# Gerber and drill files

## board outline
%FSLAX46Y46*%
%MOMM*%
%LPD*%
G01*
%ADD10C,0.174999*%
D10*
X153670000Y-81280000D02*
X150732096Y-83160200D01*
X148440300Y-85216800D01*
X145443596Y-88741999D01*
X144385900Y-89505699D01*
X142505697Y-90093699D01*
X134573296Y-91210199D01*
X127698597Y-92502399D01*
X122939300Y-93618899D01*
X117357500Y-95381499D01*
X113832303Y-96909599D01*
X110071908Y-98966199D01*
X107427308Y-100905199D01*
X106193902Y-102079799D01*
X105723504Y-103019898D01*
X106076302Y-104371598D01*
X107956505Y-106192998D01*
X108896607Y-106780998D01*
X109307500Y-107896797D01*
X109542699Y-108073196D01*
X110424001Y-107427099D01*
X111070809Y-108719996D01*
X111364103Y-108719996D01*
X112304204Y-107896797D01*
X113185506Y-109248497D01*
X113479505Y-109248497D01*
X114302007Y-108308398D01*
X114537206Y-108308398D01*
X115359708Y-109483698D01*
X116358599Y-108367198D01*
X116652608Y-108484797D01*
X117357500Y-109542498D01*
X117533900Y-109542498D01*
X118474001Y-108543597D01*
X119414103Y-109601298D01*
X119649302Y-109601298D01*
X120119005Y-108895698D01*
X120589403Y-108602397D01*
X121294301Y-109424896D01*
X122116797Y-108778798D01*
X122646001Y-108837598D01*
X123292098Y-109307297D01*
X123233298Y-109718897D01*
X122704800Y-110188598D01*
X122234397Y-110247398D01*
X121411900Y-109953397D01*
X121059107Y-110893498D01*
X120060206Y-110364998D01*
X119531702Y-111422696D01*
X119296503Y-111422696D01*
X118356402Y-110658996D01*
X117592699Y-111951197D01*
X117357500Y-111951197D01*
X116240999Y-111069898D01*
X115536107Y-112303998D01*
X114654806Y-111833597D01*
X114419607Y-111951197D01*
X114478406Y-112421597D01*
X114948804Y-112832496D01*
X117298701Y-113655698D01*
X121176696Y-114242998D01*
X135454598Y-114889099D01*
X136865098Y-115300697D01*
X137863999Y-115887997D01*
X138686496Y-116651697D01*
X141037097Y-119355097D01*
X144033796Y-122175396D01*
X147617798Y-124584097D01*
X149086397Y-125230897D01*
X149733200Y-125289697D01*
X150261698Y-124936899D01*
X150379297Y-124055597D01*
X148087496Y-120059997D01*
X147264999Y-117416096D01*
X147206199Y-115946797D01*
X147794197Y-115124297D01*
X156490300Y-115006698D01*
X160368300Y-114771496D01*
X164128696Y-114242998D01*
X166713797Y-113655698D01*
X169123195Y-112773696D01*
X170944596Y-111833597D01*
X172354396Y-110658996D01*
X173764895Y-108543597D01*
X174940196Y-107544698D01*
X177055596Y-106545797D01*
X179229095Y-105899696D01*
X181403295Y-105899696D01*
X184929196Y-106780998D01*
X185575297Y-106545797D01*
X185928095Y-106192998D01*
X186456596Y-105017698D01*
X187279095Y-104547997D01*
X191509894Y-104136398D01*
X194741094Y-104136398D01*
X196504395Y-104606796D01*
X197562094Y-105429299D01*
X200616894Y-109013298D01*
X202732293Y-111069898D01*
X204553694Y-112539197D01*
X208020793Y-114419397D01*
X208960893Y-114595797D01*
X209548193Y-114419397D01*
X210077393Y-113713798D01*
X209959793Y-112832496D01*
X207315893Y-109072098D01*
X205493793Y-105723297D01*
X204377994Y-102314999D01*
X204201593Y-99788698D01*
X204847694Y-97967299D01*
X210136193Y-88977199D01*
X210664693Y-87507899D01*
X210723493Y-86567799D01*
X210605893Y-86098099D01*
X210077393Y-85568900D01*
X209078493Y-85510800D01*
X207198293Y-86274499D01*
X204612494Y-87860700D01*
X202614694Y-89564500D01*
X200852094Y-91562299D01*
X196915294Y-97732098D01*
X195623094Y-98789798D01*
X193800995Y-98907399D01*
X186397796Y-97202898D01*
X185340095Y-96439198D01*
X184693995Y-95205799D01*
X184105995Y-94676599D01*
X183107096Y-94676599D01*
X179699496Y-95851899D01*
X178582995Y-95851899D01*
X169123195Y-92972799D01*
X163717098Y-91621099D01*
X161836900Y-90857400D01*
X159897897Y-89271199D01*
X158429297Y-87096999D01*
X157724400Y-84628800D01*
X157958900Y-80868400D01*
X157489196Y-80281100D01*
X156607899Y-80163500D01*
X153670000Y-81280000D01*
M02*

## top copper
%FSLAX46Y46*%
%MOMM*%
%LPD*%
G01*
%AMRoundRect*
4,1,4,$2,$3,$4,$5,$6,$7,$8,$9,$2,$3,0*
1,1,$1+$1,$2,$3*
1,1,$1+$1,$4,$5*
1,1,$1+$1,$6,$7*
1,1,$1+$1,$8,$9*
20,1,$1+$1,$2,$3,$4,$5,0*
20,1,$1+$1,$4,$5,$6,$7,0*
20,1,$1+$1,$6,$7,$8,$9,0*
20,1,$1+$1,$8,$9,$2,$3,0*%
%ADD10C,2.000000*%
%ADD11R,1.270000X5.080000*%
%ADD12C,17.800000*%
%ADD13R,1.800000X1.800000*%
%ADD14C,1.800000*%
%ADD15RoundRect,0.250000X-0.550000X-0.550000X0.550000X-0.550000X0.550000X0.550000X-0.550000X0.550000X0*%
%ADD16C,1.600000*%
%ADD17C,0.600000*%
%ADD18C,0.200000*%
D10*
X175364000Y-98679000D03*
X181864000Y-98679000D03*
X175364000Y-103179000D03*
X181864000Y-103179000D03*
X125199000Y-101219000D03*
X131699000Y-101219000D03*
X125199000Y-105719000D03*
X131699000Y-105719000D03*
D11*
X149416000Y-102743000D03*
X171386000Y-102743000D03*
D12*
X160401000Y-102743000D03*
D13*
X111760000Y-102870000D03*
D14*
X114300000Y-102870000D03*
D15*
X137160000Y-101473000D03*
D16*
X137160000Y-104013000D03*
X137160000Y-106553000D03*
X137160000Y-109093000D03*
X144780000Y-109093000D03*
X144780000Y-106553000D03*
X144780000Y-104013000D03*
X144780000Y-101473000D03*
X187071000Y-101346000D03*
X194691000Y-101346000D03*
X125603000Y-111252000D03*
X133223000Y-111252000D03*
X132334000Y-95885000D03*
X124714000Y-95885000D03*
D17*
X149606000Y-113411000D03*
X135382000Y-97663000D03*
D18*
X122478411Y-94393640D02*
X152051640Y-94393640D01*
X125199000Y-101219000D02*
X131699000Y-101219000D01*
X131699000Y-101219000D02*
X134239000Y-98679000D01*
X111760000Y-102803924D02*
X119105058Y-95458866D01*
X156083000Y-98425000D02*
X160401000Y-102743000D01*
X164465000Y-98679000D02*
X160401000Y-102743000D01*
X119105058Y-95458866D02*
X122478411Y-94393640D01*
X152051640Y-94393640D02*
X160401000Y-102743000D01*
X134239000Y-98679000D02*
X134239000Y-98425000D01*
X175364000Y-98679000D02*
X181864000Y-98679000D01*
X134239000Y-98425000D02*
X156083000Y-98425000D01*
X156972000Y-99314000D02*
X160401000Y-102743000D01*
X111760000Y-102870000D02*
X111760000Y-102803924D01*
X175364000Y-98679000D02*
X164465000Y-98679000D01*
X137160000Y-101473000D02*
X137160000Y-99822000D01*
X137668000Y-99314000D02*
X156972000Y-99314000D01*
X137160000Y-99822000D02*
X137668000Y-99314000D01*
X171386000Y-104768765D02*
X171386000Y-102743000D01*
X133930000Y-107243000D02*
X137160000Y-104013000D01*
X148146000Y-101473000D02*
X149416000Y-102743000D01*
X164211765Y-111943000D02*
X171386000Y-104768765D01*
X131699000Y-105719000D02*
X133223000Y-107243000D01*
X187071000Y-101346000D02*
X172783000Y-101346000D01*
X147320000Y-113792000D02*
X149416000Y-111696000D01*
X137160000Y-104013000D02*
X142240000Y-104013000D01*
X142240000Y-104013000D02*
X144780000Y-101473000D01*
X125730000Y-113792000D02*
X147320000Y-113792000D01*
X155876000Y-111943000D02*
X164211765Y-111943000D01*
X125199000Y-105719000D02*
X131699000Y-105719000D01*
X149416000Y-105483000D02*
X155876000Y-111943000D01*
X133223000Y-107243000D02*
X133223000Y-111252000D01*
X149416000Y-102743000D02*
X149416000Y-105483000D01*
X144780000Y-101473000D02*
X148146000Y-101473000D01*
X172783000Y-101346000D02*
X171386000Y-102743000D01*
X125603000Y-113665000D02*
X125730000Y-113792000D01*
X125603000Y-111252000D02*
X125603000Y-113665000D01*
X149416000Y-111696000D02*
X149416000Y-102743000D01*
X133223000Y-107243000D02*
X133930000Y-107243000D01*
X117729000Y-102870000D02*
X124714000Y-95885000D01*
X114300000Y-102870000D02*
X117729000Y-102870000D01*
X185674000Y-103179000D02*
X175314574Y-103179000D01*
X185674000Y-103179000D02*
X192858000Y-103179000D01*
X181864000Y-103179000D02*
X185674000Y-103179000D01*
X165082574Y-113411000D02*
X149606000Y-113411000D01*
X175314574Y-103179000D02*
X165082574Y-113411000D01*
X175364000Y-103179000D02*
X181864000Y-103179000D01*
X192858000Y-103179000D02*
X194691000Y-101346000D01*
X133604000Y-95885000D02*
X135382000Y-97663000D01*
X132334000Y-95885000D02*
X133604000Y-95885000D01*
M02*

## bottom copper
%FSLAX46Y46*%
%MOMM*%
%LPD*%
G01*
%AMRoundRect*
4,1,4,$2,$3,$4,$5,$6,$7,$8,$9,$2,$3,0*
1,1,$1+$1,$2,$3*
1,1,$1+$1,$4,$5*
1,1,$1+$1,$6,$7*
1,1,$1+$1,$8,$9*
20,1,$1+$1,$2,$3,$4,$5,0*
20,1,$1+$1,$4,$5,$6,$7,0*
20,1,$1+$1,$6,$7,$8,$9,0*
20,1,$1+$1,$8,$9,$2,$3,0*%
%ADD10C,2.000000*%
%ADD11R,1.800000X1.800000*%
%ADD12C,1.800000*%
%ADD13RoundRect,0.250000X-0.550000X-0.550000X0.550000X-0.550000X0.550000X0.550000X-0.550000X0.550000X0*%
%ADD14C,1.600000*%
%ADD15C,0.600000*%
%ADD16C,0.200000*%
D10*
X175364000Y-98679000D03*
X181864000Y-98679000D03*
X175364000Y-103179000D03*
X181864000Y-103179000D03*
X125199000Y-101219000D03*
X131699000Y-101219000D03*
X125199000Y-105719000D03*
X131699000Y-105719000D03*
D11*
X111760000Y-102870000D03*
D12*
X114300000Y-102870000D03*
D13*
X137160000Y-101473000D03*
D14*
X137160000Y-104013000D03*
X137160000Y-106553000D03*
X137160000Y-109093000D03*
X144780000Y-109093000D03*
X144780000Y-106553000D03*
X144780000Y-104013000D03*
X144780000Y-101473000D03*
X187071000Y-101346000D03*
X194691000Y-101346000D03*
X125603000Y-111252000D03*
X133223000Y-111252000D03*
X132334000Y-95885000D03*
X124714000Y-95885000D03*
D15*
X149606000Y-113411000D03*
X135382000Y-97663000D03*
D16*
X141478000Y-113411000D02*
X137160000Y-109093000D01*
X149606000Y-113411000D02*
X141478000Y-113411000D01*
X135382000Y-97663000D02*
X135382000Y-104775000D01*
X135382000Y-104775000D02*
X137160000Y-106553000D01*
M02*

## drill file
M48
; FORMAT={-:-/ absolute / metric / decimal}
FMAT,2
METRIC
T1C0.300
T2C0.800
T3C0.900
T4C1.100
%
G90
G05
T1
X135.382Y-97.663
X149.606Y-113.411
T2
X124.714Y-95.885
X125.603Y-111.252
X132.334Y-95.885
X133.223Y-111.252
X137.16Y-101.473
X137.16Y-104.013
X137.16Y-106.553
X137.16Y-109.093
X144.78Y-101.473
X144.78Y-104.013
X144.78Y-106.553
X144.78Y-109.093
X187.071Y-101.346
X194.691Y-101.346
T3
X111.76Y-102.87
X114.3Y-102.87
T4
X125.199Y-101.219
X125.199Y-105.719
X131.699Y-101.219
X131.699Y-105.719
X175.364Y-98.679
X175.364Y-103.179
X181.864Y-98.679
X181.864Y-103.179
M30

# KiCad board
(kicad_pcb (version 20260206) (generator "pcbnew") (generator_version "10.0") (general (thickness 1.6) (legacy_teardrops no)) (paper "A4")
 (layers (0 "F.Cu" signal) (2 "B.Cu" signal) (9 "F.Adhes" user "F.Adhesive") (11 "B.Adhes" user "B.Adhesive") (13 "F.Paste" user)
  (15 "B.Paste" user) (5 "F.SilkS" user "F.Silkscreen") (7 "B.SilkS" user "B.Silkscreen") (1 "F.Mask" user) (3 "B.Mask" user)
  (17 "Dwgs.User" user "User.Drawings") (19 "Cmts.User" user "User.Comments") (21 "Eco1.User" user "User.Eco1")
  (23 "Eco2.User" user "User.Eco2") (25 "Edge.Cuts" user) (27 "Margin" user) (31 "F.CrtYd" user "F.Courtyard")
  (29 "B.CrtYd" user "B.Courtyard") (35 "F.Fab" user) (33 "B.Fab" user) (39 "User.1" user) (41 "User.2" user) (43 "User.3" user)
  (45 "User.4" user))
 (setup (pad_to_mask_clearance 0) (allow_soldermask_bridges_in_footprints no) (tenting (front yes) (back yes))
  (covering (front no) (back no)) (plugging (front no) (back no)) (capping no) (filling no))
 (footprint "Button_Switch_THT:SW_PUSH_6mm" (layer "F.Cu") (at 175.364 98.679)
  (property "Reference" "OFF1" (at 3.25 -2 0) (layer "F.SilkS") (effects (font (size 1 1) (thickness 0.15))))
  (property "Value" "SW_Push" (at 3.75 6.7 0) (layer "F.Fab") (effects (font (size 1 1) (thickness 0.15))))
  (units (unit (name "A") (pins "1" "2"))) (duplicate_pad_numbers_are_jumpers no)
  (pad "1" thru_hole circle (at 0 0 90) (size 2 2) (drill 1.1) (layers "*.Cu" "*.Mask") (remove_unused_layers no) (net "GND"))
  (pad "1" thru_hole circle (at 6.5 0 90) (size 2 2) (drill 1.1) (layers "*.Cu" "*.Mask") (remove_unused_layers no) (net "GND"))
  (pad "2" thru_hole circle (at 0 4.5 90) (size 2 2) (drill 1.1) (layers "*.Cu" "*.Mask") (remove_unused_layers no) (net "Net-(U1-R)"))
  (pad "2" thru_hole circle (at 6.5 4.5 90) (size 2 2) (drill 1.1) (layers "*.Cu" "*.Mask") (remove_unused_layers no) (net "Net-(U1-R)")))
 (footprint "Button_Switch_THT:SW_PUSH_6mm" (layer "F.Cu") (at 125.199 101.219)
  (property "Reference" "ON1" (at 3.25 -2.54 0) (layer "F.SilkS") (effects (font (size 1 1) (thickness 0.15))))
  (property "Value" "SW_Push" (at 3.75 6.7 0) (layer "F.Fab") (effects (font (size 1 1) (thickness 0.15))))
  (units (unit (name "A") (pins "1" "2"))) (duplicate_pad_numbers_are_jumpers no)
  (pad "1" thru_hole circle (at 0 0 90) (size 2 2) (drill 1.1) (layers "*.Cu" "*.Mask") (remove_unused_layers no) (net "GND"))
  (pad "1" thru_hole circle (at 6.5 0 90) (size 2 2) (drill 1.1) (layers "*.Cu" "*.Mask") (remove_unused_layers no) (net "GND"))
  (pad "2" thru_hole circle (at 0 4.5 90) (size 2 2) (drill 1.1) (layers "*.Cu" "*.Mask") (remove_unused_layers no) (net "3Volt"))
  (pad "2" thru_hole circle (at 6.5 4.5 90) (size 2 2) (drill 1.1) (layers "*.Cu" "*.Mask") (remove_unused_layers no) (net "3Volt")))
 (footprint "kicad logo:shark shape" (layer "F.Cu") (at 124.714 104.267 180)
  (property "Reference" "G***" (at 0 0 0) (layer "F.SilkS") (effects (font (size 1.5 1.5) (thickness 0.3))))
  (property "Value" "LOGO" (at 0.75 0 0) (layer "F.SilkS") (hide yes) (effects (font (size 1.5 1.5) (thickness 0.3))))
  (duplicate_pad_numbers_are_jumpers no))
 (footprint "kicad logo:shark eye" (layer "F.Cu") (at 113.831779 99.989505 65)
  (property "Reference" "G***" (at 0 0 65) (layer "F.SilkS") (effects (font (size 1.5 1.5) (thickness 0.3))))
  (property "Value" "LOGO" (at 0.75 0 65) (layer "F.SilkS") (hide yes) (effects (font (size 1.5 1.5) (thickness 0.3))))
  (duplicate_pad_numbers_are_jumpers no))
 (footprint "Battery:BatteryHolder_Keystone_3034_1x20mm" (layer "F.Cu") (at 160.401 102.743)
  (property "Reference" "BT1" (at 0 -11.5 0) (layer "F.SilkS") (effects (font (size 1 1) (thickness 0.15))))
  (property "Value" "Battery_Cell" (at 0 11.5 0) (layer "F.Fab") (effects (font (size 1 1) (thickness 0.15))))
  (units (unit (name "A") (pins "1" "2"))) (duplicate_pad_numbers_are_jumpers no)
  (pad "1" smd rect (at -10.985 0) (size 1.27 5.08) (layers "F.Cu" "F.Mask" "F.Paste") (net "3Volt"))
  (pad "1" smd rect (at 10.985 0) (size 1.27 5.08) (layers "F.Cu" "F.Mask" "F.Paste") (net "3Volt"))
  (pad "2" smd circle (at 0 0) (size 17.8 17.8) (layers "F.Cu" "F.Mask") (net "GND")))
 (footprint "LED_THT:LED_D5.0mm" (layer "F.Cu") (at 111.76 102.87)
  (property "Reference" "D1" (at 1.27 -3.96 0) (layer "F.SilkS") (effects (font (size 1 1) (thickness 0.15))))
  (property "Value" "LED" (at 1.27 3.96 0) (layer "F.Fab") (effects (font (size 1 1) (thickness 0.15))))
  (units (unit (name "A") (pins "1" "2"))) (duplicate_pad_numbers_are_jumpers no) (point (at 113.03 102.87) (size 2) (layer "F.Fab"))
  (pad "1" thru_hole rect (at 0 0) (size 1.8 1.8) (drill 0.9) (layers "*.Cu" "*.Mask") (remove_unused_layers no) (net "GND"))
  (pad "2" thru_hole circle (at 2.54 0) (size 1.8 1.8) (drill 0.9) (layers "*.Cu" "*.Mask") (remove_unused_layers no) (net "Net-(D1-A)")))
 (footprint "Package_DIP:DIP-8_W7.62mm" (layer "F.Cu") (at 137.16 101.473)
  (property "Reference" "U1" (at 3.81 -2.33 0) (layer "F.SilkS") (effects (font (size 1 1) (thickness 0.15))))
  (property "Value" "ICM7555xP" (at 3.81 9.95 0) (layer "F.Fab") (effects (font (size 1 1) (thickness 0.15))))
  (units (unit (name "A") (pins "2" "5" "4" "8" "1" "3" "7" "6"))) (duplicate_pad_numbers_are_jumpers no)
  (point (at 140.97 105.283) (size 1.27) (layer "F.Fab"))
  (pad "1" thru_hole roundrect (at 0 0) (size 1.6 1.6) (drill 0.8) (layers "*.Cu" "*.Mask") (remove_unused_layers no)
   (roundrect_rratio 0.15625) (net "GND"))
  (pad "2" thru_hole circle (at 0 2.54) (size 1.6 1.6) (drill 0.8) (layers "*.Cu" "*.Mask") (remove_unused_layers no) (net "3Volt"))
  (pad "3" thru_hole circle (at 0 5.08) (size 1.6 1.6) (drill 0.8) (layers "*.Cu" "*.Mask") (remove_unused_layers no) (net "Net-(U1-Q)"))
  (pad "4" thru_hole circle (at 0 7.62) (size 1.6 1.6) (drill 0.8) (layers "*.Cu" "*.Mask") (remove_unused_layers no) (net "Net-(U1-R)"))
  (pad "5" thru_hole circle (at 7.62 7.62) (size 1.6 1.6) (drill 0.8) (layers "*.Cu" "*.Mask") (remove_unused_layers no)
   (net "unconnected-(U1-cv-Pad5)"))
  (pad "6" thru_hole circle (at 7.62 5.08) (size 1.6 1.6) (drill 0.8) (layers "*.Cu" "*.Mask") (remove_unused_layers no)
   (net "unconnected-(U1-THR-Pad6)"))
  (pad "7" thru_hole circle (at 7.62 2.54) (size 1.6 1.6) (drill 0.8) (layers "*.Cu" "*.Mask") (remove_unused_layers no)
   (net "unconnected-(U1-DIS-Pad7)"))
  (pad "8" thru_hole circle (at 7.62 0) (size 1.6 1.6) (drill 0.8) (layers "*.Cu" "*.Mask") (remove_unused_layers no) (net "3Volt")))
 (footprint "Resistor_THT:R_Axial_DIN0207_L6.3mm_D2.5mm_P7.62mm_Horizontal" (layer "F.Cu") (at 187.071 101.346)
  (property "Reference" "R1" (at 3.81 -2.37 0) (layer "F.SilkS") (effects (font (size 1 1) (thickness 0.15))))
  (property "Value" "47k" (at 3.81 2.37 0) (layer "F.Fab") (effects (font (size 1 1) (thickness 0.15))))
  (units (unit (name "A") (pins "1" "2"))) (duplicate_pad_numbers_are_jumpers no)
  (pad "1" thru_hole circle (at 0 0) (size 1.6 1.6) (drill 0.8) (layers "*.Cu" "*.Mask") (remove_unused_layers no) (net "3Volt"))
  (pad "2" thru_hole circle (at 7.62 0) (size 1.6 1.6) (drill 0.8) (layers "*.Cu" "*.Mask") (remove_unused_layers no) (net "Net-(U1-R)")))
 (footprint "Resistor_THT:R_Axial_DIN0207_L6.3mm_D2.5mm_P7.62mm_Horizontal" (layer "F.Cu") (at 125.603 111.252)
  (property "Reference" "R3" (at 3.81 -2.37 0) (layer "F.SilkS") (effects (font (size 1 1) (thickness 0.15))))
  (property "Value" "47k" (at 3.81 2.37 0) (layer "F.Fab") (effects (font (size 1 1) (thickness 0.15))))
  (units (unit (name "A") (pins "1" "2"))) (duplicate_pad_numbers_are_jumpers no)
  (pad "1" thru_hole circle (at 0 0) (size 1.6 1.6) (drill 0.8) (layers "*.Cu" "*.Mask") (remove_unused_layers no) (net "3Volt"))
  (pad "2" thru_hole circle (at 7.62 0) (size 1.6 1.6) (drill 0.8) (layers "*.Cu" "*.Mask") (remove_unused_layers no) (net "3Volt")))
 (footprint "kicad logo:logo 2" (layer "F.Cu") (at 151.511 90.17 50)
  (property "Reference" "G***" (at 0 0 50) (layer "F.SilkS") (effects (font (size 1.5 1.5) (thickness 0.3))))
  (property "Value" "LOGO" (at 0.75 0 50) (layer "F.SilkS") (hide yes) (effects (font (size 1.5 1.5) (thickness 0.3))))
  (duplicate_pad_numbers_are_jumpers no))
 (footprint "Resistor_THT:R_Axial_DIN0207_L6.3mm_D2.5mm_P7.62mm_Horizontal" (layer "F.Cu") (at 132.334 95.885 180)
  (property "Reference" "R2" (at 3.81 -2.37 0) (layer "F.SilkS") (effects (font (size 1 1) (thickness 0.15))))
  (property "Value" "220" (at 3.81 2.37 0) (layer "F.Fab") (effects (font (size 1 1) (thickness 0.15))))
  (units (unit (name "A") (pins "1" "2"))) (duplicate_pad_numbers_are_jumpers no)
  (pad "1" thru_hole circle (at 0 0 180) (size 1.6 1.6) (drill 0.8) (layers "*.Cu" "*.Mask") (remove_unused_layers no) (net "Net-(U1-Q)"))
  (pad "2" thru_hole circle (at 7.62 0 180) (size 1.6 1.6) (drill 0.8) (layers "*.Cu" "*.Mask") (remove_unused_layers no) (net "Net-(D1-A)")))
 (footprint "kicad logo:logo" (layer "B.Cu") (at 155.956 102.743 180)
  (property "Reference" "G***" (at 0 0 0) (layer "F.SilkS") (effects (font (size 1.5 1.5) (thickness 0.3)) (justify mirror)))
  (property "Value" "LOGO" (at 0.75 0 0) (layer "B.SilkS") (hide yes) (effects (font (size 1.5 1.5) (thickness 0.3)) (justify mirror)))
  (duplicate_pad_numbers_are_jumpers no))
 (gr_poly
  (pts (xy 153.67 81.28) (xy 150.732096 83.1602) (xy 148.4403 85.2168) (xy 145.443596 88.741999) (xy 144.3859 89.505699)
   (xy 142.505697 90.093699) (xy 134.573296 91.210199) (xy 127.698597 92.502399) (xy 122.9393 93.618899) (xy 117.3575 95.381499)
   (xy 113.832303 96.909599) (xy 110.071908 98.966199) (xy 107.427308 100.905199) (xy 106.193902 102.079799) (xy 105.723504 103.019898)
   (xy 106.076302 104.371598) (xy 107.956505 106.192998) (xy 108.896607 106.780998) (xy 109.3075 107.896797) (xy 109.542699 108.073196)
   (xy 110.424001 107.427099) (xy 111.070809 108.719996) (xy 111.364103 108.719996) (xy 112.304204 107.896797) (xy 113.185506 109.248497)
   (xy 113.479505 109.248497) (xy 114.302007 108.308398) (xy 114.537206 108.308398) (xy 115.359708 109.483698) (xy 116.358599 108.367198)
   (xy 116.652608 108.484797) (xy 117.3575 109.542498) (xy 117.5339 109.542498) (xy 118.474001 108.543597) (xy 119.414103 109.601298)
   (xy 119.649302 109.601298) (xy 120.119005 108.895698) (xy 120.589403 108.602397) (xy 121.294301 109.424896) (xy 122.116797 108.778798)
   (xy 122.646001 108.837598) (xy 123.292098 109.307297) (xy 123.233298 109.718897) (xy 122.7048 110.188598) (xy 122.234397 110.247398)
   (xy 121.4119 109.953397) (xy 121.059107 110.893498) (xy 120.060206 110.364998) (xy 119.531702 111.422696) (xy 119.296503 111.422696)
   (xy 118.356402 110.658996) (xy 117.592699 111.951197) (xy 117.3575 111.951197) (xy 116.240999 111.069898) (xy 115.536107 112.303998)
   (xy 114.654806 111.833597) (xy 114.419607 111.951197) (xy 114.478406 112.421597) (xy 114.948804 112.832496) (xy 117.298701 113.655698)
   (xy 121.176696 114.242998) (xy 135.454598 114.889099) (xy 136.865098 115.300697) (xy 137.863999 115.887997) (xy 138.686496 116.651697)
   (xy 141.037097 119.355097) (xy 144.033796 122.175396) (xy 147.617798 124.584097) (xy 149.086397 125.230897) (xy 149.7332 125.289697)
   (xy 150.261698 124.936899) (xy 150.379297 124.055597) (xy 148.087496 120.059997) (xy 147.264999 117.416096) (xy 147.206199 115.946797)
   (xy 147.794197 115.124297) (xy 156.4903 115.006698) (xy 160.3683 114.771496) (xy 164.128696 114.242998) (xy 166.713797 113.655698)
   (xy 169.123195 112.773696) (xy 170.944596 111.833597) (xy 172.354396 110.658996) (xy 173.764895 108.543597) (xy 174.940196 107.544698)
   (xy 177.055596 106.545797) (xy 179.229095 105.899696) (xy 181.403295 105.899696) (xy 184.929196 106.780998) (xy 185.575297 106.545797)
   (xy 185.928095 106.192998) (xy 186.456596 105.017698) (xy 187.279095 104.547997) (xy 191.509894 104.136398) (xy 194.741094 104.136398)
   (xy 196.504395 104.606796) (xy 197.562094 105.429299) (xy 200.616894 109.013298) (xy 202.732293 111.069898) (xy 204.553694 112.539197)
   (xy 208.020793 114.419397) (xy 208.960893 114.595797) (xy 209.548193 114.419397) (xy 210.077393 113.713798) (xy 209.959793 112.832496)
   (xy 207.315893 109.072098) (xy 205.493793 105.723297) (xy 204.377994 102.314999) (xy 204.201593 99.788698) (xy 204.847694 97.967299)
   (xy 210.136193 88.977199) (xy 210.664693 87.507899) (xy 210.723493 86.567799) (xy 210.605893 86.098099) (xy 210.077393 85.5689)
   (xy 209.078493 85.5108) (xy 207.198293 86.274499) (xy 204.612494 87.8607) (xy 202.614694 89.5645) (xy 200.852094 91.562299)
   (xy 196.915294 97.732098) (xy 195.623094 98.789798) (xy 193.800995 98.907399) (xy 186.397796 97.202898) (xy 185.340095 96.439198)
   (xy 184.693995 95.205799) (xy 184.105995 94.676599) (xy 183.107096 94.676599) (xy 179.699496 95.851899) (xy 178.582995 95.851899)
   (xy 169.123195 92.972799) (xy 163.717098 91.621099) (xy 161.8369 90.8574) (xy 159.897897 89.271199) (xy 158.429297 87.096999)
   (xy 157.7244 84.6288) (xy 157.9589 80.8684) (xy 157.489196 80.2811) (xy 156.607899 80.1635))
  (stroke (width 0.174999) (type solid)) (fill no) (layer "Edge.Cuts"))
 (segment (start 122.478411 94.39364) (end 152.05164 94.39364) (width 0.2) (layer "F.Cu") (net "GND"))
 (segment (start 125.199 101.219) (end 131.699 101.219) (width 0.2) (layer "F.Cu") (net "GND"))
 (segment (start 131.699 101.219) (end 134.239 98.679) (width 0.2) (layer "F.Cu") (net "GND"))
 (segment (start 111.76 102.803924) (end 119.105058 95.458866) (width 0.2) (layer "F.Cu") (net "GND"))
 (segment (start 156.083 98.425) (end 160.401 102.743) (width 0.2) (layer "F.Cu") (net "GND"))
 (segment (start 164.465 98.679) (end 160.401 102.743) (width 0.2) (layer "F.Cu") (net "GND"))
 (segment (start 119.105058 95.458866) (end 122.478411 94.39364) (width 0.2) (layer "F.Cu") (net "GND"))
 (segment (start 152.05164 94.39364) (end 160.401 102.743) (width 0.2) (layer "F.Cu") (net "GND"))
 (segment (start 134.239 98.679) (end 134.239 98.425) (width 0.2) (layer "F.Cu") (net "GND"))
 (segment (start 175.364 98.679) (end 181.864 98.679) (width 0.2) (layer "F.Cu") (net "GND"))
 (segment (start 134.239 98.425) (end 156.083 98.425) (width 0.2) (layer "F.Cu") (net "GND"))
 (segment (start 156.972 99.314) (end 160.401 102.743) (width 0.2) (layer "F.Cu") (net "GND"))
 (segment (start 111.76 102.87) (end 111.76 102.803924) (width 0.2) (layer "F.Cu") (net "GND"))
 (segment (start 175.364 98.679) (end 164.465 98.679) (width 0.2) (layer "F.Cu") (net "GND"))
 (segment (start 137.16 101.473) (end 137.16 99.822) (width 0.2) (layer "F.Cu") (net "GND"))
 (segment (start 137.668 99.314) (end 156.972 99.314) (width 0.2) (layer "F.Cu") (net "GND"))
 (segment (start 137.16 99.822) (end 137.668 99.314) (width 0.2) (layer "F.Cu") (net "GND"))
 (segment (start 171.386 104.768765) (end 171.386 102.743) (width 0.2) (layer "F.Cu") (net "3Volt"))
 (segment (start 133.93 107.243) (end 137.16 104.013) (width 0.2) (layer "F.Cu") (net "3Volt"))
 (segment (start 148.146 101.473) (end 149.416 102.743) (width 0.2) (layer "F.Cu") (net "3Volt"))
 (segment (start 164.211765 111.943) (end 171.386 104.768765) (width 0.2) (layer "F.Cu") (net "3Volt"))
 (segment (start 131.699 105.719) (end 133.223 107.243) (width 0.2) (layer "F.Cu") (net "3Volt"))
 (segment (start 187.071 101.346) (end 172.783 101.346) (width 0.2) (layer "F.Cu") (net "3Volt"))
 (segment (start 147.32 113.792) (end 149.416 111.696) (width 0.2) (layer "F.Cu") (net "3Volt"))
 (segment (start 137.16 104.013) (end 142.24 104.013) (width 0.2) (layer "F.Cu") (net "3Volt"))
 (segment (start 142.24 104.013) (end 144.78 101.473) (width 0.2) (layer "F.Cu") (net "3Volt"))
 (segment (start 125.73 113.792) (end 147.32 113.792) (width 0.2) (layer "F.Cu") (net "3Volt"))
 (segment (start 155.876 111.943) (end 164.211765 111.943) (width 0.2) (layer "F.Cu") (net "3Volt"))
 (segment (start 125.199 105.719) (end 131.699 105.719) (width 0.2) (layer "F.Cu") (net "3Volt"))
 (segment (start 149.416 105.483) (end 155.876 111.943) (width 0.2) (layer "F.Cu") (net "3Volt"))
 (segment (start 133.223 107.243) (end 133.223 111.252) (width 0.2) (layer "F.Cu") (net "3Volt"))
 (segment (start 149.416 102.743) (end 149.416 105.483) (width 0.2) (layer "F.Cu") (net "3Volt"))
 (segment (start 144.78 101.473) (end 148.146 101.473) (width 0.2) (layer "F.Cu") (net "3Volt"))
 (segment (start 172.783 101.346) (end 171.386 102.743) (width 0.2) (layer "F.Cu") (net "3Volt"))
 (segment (start 125.603 113.665) (end 125.73 113.792) (width 0.2) (layer "F.Cu") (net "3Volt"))
 (segment (start 125.603 111.252) (end 125.603 113.665) (width 0.2) (layer "F.Cu") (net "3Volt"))
 (segment (start 149.416 111.696) (end 149.416 102.743) (width 0.2) (layer "F.Cu") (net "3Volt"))
 (segment (start 133.223 107.243) (end 133.93 107.243) (width 0.2) (layer "F.Cu") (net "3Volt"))
 (segment (start 117.729 102.87) (end 124.714 95.885) (width 0.2) (layer "F.Cu") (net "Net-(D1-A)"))
 (segment (start 114.3 102.87) (end 117.729 102.87) (width 0.2) (layer "F.Cu") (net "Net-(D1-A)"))
 (segment (start 185.674 103.179) (end 175.314574 103.179) (width 0.2) (layer "F.Cu") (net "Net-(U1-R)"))
 (segment (start 185.674 103.179) (end 192.858 103.179) (width 0.2) (layer "F.Cu") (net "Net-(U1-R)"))
 (segment (start 181.864 103.179) (end 185.674 103.179) (width 0.2) (layer "F.Cu") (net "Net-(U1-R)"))
 (segment (start 165.082574 113.411) (end 149.606 113.411) (width 0.2) (layer "F.Cu") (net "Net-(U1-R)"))
 (segment (start 175.314574 103.179) (end 165.082574 113.411) (width 0.2) (layer "F.Cu") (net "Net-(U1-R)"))
 (segment (start 175.364 103.179) (end 181.864 103.179) (width 0.2) (layer "F.Cu") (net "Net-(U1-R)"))
 (segment (start 192.858 103.179) (end 194.691 101.346) (width 0.2) (layer "F.Cu") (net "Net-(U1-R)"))
 (via (at 149.606 113.411) (size 0.6) (drill 0.3) (layers "F.Cu" "B.Cu") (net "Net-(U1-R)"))
 (segment (start 141.478 113.411) (end 137.16 109.093) (width 0.2) (layer "B.Cu") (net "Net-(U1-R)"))
 (segment (start 149.606 113.411) (end 141.478 113.411) (width 0.2) (layer "B.Cu") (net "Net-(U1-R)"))
 (segment (start 133.604 95.885) (end 135.382 97.663) (width 0.2) (layer "F.Cu") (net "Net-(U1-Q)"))
 (segment (start 132.334 95.885) (end 133.604 95.885) (width 0.2) (layer "F.Cu") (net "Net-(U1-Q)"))
 (via (at 135.382 97.663) (size 0.6) (drill 0.3) (layers "F.Cu" "B.Cu") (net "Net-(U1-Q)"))
 (segment (start 135.382 97.663) (end 135.382 104.775) (width 0.2) (layer "B.Cu") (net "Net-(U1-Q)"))
 (segment (start 135.382 104.775) (end 137.16 106.553) (width 0.2) (layer "B.Cu") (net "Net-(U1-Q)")))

